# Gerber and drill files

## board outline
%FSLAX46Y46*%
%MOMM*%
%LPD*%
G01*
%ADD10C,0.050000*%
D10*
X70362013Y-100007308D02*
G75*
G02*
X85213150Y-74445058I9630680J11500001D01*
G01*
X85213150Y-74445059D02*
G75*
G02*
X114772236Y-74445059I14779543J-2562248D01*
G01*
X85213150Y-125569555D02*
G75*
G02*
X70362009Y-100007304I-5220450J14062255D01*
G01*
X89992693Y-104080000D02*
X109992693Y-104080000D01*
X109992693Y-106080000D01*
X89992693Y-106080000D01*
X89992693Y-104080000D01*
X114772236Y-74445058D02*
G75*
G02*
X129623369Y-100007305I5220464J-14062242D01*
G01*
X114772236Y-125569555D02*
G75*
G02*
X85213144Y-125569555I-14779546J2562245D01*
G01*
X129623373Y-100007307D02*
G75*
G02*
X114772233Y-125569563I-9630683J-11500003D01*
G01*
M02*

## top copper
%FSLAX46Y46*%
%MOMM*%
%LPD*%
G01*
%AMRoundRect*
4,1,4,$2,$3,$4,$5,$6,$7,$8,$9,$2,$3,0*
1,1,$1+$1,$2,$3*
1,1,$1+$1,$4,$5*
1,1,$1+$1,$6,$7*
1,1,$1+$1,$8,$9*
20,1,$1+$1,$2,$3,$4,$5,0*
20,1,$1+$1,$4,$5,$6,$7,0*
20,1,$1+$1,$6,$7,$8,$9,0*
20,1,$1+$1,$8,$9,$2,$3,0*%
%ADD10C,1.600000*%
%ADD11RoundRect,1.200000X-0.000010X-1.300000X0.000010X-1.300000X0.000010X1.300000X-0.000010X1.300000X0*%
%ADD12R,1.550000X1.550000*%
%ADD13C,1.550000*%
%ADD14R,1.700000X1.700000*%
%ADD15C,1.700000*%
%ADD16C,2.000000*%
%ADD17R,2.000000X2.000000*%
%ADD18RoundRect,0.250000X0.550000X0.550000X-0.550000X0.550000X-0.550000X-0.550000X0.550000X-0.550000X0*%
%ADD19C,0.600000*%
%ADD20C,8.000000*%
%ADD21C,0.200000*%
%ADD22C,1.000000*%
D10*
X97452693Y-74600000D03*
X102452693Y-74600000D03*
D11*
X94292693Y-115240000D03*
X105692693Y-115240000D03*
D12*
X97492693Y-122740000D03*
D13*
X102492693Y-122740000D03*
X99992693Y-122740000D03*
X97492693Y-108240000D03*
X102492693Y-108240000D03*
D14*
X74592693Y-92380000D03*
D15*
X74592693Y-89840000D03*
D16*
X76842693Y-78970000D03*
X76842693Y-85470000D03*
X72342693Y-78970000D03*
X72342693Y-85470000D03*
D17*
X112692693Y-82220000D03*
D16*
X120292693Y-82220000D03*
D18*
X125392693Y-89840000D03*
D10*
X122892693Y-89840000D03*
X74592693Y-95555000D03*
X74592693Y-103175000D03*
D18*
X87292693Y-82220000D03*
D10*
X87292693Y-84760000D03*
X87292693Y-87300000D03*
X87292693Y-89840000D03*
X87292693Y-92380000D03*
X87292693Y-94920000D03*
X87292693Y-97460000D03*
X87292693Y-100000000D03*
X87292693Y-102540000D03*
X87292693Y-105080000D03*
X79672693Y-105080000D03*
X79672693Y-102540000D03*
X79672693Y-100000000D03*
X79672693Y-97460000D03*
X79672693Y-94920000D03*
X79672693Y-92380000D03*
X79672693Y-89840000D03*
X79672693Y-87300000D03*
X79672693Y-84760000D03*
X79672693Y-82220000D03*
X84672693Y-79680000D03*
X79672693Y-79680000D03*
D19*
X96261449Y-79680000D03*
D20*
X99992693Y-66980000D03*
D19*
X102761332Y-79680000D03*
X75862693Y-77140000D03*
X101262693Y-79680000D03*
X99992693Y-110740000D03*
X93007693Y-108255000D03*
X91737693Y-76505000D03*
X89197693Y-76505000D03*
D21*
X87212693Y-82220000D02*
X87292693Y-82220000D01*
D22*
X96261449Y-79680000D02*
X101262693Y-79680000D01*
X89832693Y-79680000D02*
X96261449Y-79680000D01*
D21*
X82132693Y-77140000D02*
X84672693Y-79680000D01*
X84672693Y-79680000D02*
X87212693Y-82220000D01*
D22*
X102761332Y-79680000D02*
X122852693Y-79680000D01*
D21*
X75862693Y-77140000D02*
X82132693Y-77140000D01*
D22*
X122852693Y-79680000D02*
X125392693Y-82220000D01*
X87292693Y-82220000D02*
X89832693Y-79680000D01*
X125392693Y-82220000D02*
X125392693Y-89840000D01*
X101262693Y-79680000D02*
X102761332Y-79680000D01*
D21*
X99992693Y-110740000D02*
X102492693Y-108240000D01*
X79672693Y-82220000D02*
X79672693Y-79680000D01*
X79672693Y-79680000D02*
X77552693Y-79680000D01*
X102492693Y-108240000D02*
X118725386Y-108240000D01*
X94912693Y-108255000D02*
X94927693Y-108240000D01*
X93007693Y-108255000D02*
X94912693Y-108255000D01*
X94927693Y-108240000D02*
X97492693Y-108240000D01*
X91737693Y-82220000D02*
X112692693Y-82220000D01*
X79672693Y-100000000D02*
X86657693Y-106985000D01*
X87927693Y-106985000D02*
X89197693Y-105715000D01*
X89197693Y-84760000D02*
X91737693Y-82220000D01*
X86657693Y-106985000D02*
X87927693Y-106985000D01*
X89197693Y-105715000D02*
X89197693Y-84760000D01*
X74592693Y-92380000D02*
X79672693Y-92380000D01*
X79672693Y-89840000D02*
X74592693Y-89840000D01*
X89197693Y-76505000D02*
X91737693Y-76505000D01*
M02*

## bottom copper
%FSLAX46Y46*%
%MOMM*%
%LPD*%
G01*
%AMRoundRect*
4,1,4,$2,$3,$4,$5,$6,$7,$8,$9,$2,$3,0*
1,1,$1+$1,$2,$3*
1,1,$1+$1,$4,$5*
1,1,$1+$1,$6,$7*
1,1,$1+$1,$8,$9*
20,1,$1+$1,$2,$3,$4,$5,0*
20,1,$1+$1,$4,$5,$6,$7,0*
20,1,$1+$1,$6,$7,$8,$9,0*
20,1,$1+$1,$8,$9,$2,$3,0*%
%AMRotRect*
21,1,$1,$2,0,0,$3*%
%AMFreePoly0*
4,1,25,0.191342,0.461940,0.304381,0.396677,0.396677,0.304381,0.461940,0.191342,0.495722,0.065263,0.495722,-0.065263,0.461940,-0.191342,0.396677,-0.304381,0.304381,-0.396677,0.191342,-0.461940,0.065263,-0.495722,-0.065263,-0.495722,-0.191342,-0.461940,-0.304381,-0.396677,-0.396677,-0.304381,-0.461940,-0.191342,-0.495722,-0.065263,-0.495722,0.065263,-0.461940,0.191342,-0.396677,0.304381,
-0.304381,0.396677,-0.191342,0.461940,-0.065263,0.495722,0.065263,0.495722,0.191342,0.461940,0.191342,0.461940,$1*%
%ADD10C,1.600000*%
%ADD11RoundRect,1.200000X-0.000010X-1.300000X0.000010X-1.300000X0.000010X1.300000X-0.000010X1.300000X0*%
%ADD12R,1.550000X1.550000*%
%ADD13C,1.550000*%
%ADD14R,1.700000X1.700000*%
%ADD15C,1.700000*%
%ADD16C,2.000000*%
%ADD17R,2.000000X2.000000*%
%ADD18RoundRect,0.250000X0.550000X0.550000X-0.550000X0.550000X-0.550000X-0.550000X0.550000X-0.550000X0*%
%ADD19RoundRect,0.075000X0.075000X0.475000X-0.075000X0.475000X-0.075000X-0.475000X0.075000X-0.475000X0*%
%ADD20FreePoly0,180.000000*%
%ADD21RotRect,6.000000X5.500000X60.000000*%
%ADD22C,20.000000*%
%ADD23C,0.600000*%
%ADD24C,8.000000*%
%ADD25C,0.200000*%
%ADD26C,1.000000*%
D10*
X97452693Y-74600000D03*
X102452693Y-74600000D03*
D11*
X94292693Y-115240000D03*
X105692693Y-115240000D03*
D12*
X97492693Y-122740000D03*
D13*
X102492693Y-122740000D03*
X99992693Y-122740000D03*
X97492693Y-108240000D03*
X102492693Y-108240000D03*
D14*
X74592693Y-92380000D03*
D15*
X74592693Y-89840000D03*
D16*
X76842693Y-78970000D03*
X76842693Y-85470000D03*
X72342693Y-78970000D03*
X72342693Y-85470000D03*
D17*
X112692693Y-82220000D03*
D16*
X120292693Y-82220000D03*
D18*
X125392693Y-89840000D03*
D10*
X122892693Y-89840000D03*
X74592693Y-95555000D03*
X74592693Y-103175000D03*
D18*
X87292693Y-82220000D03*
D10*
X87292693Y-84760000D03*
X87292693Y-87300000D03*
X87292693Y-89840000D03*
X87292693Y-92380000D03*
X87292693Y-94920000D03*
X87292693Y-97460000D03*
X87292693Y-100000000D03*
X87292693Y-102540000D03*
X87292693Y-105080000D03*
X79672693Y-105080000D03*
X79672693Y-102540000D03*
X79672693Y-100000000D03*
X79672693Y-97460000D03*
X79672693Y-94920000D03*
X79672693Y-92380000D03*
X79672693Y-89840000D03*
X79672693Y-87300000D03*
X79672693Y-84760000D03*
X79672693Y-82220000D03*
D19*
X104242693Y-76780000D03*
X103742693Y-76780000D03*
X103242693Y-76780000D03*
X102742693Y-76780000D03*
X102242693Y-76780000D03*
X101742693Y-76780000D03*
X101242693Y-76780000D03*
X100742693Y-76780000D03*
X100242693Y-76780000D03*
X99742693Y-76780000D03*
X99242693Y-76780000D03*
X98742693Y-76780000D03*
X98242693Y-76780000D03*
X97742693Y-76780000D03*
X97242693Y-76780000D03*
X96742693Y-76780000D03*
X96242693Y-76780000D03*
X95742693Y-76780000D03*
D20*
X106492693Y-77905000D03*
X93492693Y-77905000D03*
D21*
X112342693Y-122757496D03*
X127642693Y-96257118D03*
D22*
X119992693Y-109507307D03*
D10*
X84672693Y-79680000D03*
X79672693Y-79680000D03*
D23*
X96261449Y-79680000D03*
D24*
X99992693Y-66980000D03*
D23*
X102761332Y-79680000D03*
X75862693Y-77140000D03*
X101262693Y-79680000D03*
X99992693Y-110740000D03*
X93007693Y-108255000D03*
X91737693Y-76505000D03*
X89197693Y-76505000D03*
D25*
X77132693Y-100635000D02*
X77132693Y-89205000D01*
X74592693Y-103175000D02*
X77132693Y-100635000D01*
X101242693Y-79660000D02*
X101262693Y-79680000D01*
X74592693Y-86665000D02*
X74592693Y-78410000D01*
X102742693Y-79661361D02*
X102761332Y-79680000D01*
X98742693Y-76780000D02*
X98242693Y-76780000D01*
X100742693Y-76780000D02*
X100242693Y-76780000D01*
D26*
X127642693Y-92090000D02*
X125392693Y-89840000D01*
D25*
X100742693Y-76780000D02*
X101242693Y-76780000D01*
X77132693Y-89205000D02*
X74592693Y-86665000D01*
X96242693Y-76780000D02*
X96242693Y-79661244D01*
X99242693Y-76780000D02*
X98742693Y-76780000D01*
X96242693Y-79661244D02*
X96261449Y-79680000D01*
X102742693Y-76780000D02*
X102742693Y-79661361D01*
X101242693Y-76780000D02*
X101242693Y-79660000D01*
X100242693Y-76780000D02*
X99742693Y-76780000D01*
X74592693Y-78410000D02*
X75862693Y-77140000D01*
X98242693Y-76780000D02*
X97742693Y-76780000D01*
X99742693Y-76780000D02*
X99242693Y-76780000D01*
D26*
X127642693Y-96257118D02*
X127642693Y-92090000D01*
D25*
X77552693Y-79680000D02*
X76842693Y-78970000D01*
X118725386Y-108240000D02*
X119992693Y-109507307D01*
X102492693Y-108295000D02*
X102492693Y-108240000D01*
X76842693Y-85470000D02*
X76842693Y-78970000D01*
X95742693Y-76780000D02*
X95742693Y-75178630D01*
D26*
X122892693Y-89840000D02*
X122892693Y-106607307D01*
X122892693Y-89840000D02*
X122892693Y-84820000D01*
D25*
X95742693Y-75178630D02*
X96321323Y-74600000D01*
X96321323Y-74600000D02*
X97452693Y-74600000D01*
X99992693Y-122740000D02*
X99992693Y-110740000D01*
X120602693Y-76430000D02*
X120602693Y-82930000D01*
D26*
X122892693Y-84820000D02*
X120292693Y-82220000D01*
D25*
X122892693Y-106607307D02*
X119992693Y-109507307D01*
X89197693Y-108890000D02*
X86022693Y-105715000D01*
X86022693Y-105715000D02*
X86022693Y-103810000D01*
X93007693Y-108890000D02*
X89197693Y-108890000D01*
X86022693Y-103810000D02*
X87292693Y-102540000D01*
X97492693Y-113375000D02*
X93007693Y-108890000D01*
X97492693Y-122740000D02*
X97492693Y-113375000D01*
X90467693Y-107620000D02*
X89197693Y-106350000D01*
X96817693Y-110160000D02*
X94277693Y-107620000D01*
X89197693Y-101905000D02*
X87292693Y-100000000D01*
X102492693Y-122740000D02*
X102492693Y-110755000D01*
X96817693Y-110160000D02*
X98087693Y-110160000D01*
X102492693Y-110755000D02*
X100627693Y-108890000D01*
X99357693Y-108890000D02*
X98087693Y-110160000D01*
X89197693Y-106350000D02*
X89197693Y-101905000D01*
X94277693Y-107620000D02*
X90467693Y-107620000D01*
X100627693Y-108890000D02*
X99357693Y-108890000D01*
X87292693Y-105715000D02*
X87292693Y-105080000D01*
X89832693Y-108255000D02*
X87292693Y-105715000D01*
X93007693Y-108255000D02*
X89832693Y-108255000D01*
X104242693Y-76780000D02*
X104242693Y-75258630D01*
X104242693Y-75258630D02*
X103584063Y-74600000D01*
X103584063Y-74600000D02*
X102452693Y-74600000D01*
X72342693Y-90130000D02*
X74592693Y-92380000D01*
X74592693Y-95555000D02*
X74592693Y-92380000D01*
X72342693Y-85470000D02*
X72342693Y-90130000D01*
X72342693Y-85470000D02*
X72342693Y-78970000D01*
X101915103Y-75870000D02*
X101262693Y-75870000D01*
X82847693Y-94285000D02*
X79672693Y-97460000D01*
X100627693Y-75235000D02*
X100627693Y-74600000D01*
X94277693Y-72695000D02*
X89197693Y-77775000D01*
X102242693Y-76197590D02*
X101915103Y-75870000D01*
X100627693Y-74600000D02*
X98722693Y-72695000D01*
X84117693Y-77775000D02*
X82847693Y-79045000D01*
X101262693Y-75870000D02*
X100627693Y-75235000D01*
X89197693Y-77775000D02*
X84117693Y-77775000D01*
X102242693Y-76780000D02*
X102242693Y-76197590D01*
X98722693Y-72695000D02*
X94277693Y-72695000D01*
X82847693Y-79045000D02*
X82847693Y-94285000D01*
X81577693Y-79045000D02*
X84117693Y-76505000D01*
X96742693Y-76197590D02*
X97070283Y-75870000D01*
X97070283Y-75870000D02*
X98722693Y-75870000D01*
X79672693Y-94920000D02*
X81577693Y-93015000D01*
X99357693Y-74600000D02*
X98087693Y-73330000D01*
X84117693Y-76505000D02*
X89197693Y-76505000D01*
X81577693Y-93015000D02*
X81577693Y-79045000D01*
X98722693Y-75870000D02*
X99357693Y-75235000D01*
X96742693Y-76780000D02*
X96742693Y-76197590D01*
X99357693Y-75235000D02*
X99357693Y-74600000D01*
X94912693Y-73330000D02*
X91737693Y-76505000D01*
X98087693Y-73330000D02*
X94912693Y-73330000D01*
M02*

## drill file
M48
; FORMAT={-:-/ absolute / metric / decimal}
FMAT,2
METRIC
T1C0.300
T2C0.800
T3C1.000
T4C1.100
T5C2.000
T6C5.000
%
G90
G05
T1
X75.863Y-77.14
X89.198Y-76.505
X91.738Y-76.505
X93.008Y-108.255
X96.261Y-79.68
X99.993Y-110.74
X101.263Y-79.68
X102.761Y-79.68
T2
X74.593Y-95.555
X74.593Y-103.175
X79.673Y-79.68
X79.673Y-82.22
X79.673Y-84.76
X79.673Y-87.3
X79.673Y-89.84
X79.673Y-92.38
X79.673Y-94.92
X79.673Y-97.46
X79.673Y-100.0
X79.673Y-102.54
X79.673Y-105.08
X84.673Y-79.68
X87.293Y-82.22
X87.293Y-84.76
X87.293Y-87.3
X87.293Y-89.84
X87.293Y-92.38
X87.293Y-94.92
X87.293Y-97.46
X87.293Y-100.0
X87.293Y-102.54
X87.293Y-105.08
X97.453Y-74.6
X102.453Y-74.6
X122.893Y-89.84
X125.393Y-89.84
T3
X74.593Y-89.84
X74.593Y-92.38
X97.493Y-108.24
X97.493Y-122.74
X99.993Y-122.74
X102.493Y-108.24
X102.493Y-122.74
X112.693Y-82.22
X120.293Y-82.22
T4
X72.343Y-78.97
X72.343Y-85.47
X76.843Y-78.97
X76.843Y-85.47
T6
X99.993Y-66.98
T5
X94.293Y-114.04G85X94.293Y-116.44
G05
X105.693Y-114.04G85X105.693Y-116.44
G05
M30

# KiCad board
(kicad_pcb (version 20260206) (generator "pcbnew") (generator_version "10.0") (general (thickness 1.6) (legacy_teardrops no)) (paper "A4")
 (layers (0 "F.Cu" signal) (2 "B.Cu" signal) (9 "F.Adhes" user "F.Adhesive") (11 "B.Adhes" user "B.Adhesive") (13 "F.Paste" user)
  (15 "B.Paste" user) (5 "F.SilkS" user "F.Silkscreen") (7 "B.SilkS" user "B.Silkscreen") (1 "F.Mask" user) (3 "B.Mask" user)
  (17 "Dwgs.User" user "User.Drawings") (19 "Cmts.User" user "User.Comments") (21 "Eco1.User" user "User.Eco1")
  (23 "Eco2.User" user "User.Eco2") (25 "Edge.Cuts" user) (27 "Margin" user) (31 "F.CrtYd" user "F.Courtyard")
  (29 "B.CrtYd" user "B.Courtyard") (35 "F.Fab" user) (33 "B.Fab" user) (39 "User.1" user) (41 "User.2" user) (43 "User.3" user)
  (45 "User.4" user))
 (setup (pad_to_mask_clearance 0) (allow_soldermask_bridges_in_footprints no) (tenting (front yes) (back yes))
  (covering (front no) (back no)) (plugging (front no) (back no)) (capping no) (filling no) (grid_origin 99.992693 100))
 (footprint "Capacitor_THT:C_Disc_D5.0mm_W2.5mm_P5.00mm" (layer "F.Cu") (at 97.452693 74.6)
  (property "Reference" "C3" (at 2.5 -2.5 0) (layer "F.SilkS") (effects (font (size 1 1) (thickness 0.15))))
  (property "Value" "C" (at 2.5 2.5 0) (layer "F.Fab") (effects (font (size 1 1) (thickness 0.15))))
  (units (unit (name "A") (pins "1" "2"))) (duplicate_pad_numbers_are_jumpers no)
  (pad "1" thru_hole circle (at 0 0) (size 1.6 1.6) (drill 0.8) (layers "*.Cu" "*.Mask") (remove_unused_layers no) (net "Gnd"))
  (pad "2" thru_hole circle (at 5 0) (size 1.6 1.6) (drill 0.8) (layers "*.Cu" "*.Mask") (remove_unused_layers no) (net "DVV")))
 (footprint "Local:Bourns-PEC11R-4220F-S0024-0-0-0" (layer "F.Cu") (at 99.992693 115.24)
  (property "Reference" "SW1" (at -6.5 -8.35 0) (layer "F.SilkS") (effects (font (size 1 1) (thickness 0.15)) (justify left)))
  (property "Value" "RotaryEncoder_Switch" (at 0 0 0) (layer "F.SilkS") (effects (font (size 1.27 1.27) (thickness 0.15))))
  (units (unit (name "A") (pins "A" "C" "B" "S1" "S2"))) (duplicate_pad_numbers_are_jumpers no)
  (pad "3" thru_hole roundrect (at -5.7 0) (size 2.4 5) (drill oval 2 4.4) (layers "*.Cu" "*.Mask") (remove_unused_layers no)
   (roundrect_rratio 0.5))
  (pad "4" thru_hole roundrect (at 5.7 0) (size 2.4 5) (drill oval 2 4.4) (layers "*.Cu" "*.Mask") (remove_unused_layers no)
   (roundrect_rratio 0.5))
  (pad "A" thru_hole rect (at -2.5 7.5) (size 1.55 1.55) (drill 1) (layers "*.Cu" "*.Mask") (remove_unused_layers no) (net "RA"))
  (pad "B" thru_hole circle (at 2.5 7.5) (size 1.55 1.55) (drill 1) (layers "*.Cu" "*.Mask") (remove_unused_layers no) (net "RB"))
  (pad "C" thru_hole circle (at 0 7.5) (size 1.55 1.55) (drill 1) (layers "*.Cu" "*.Mask") (remove_unused_layers no) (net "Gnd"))
  (pad "S1" thru_hole circle (at -2.5 -7) (size 1.55 1.55) (drill 1) (layers "*.Cu" "*.Mask") (remove_unused_layers no) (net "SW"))
  (pad "S2" thru_hole circle (at 2.5 -7) (size 1.55 1.55) (drill 1) (layers "*.Cu" "*.Mask") (remove_unused_layers no) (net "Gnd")))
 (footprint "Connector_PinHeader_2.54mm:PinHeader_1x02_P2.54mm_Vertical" (layer "F.Cu") (at 74.592693 92.38 180)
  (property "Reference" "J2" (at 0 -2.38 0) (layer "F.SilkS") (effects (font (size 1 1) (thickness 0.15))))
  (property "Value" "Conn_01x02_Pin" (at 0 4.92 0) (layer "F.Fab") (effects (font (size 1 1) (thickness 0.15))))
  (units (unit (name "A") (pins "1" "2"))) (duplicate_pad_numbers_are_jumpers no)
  (pad "1" thru_hole rect (at 0 0 180) (size 1.7 1.7) (drill 1) (layers "*.Cu" "*.Mask") (remove_unused_layers no) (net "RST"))
  (pad "2" thru_hole circle (at 0 2.54 180) (size 1.7 1.7) (drill 1) (layers "*.Cu" "*.Mask") (remove_unused_layers no) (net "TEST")))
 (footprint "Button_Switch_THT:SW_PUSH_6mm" (layer "F.Cu") (at 76.842693 78.97 -90)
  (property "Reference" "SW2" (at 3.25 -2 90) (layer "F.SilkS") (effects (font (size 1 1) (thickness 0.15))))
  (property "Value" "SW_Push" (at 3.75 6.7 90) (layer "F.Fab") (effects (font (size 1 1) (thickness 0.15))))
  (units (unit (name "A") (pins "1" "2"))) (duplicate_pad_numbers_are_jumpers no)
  (pad "1" thru_hole circle (at 0 0) (size 2 2) (drill 1.1) (layers "*.Cu" "*.Mask") (remove_unused_layers no) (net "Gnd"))
  (pad "1" thru_hole circle (at 6.5 0) (size 2 2) (drill 1.1) (layers "*.Cu" "*.Mask") (remove_unused_layers no) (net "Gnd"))
  (pad "2" thru_hole circle (at 0 4.5) (size 2 2) (drill 1.1) (layers "*.Cu" "*.Mask") (remove_unused_layers no) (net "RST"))
  (pad "2" thru_hole circle (at 6.5 4.5) (size 2 2) (drill 1.1) (layers "*.Cu" "*.Mask") (remove_unused_layers no) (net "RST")))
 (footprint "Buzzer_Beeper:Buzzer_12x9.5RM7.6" (layer "F.Cu") (at 112.692693 82.22)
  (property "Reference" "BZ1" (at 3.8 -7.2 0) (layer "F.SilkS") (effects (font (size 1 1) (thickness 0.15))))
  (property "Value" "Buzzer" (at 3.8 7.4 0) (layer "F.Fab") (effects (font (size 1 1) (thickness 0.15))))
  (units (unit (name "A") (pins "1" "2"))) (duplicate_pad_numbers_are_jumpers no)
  (pad "1" thru_hole rect (at 0 0) (size 2 2) (drill 1) (layers "*.Cu" "*.Mask") (remove_unused_layers no) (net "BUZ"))
  (pad "2" thru_hole circle (at 7.6 0) (size 2 2) (drill 1) (layers "*.Cu" "*.Mask") (remove_unused_layers no) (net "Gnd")))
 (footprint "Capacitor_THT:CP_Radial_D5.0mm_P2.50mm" (layer "F.Cu") (at 125.392693 89.84 180)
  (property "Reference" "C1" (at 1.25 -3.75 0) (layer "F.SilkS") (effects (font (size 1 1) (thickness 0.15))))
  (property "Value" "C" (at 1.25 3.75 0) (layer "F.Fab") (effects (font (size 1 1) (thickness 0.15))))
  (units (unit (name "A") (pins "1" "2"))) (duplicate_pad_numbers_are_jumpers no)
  (pad "1" thru_hole roundrect (at 0 0 180) (size 1.6 1.6) (drill 0.8) (layers "*.Cu" "*.Mask") (remove_unused_layers no)
   (roundrect_rratio 0.15625) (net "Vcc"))
  (pad "2" thru_hole circle (at 2.5 0 180) (size 1.6 1.6) (drill 0.8) (layers "*.Cu" "*.Mask") (remove_unused_layers no) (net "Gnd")))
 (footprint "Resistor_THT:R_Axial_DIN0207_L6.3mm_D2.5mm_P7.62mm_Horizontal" (layer "F.Cu") (at 74.592693 95.555 -90)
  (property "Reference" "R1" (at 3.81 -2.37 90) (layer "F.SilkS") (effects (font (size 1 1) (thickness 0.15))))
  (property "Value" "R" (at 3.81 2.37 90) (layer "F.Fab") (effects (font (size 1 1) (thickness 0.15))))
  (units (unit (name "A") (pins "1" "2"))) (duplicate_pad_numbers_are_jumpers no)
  (pad "1" thru_hole circle (at 0 0 270) (size 1.6 1.6) (drill 0.8) (layers "*.Cu" "*.Mask") (remove_unused_layers no) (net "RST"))
  (pad "2" thru_hole circle (at 7.62 0 270) (size 1.6 1.6) (drill 0.8) (layers "*.Cu" "*.Mask") (remove_unused_layers no) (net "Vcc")))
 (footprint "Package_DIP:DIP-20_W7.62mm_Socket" (layer "B.Cu") (at 87.292693 82.22 180)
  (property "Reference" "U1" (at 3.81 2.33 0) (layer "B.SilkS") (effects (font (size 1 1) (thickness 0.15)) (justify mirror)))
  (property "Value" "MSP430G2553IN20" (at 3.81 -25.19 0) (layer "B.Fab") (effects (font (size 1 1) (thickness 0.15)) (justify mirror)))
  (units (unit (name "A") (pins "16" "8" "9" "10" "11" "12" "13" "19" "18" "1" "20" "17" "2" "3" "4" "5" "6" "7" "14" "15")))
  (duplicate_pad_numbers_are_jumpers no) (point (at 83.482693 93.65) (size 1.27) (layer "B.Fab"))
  (pad "1" thru_hole roundrect (at 0 0 180) (size 1.6 1.6) (drill 0.8) (layers "*.Cu" "*.Mask") (remove_unused_layers no)
   (roundrect_rratio 0.15625) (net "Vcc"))
  (pad "2" thru_hole circle (at 0 -2.54 180) (size 1.6 1.6) (drill 0.8) (layers "*.Cu" "*.Mask") (remove_unused_layers no)
   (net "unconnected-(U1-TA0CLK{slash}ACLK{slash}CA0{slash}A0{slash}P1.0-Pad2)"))
  (pad "3" thru_hole circle (at 0 -5.08 180) (size 1.6 1.6) (drill 0.8) (layers "*.Cu" "*.Mask") (remove_unused_layers no)
   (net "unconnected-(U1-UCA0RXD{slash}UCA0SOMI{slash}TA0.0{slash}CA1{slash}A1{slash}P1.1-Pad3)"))
  (pad "4" thru_hole circle (at 0 -7.62 180) (size 1.6 1.6) (drill 0.8) (layers "*.Cu" "*.Mask") (remove_unused_layers no) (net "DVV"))
  (pad "5" thru_hole circle (at 0 -10.16 180) (size 1.6 1.6) (drill 0.8) (layers "*.Cu" "*.Mask") (remove_unused_layers no) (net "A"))
  (pad "6" thru_hole circle (at 0 -12.7 180) (size 1.6 1.6) (drill 0.8) (layers "*.Cu" "*.Mask") (remove_unused_layers no) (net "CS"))
  (pad "7" thru_hole circle (at 0 -15.24 180) (size 1.6 1.6) (drill 0.8) (layers "*.Cu" "*.Mask") (remove_unused_layers no) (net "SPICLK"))
  (pad "8" thru_hole circle (at 0 -17.78 180) (size 1.6 1.6) (drill 0.8) (layers "*.Cu" "*.Mask") (remove_unused_layers no) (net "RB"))
  (pad "9" thru_hole circle (at 0 -20.32 180) (size 1.6 1.6) (drill 0.8) (layers "*.Cu" "*.Mask") (remove_unused_layers no) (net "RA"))
  (pad "10" thru_hole circle (at 0 -22.86 180) (size 1.6 1.6) (drill 0.8) (layers "*.Cu" "*.Mask") (remove_unused_layers no) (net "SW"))
  (pad "11" thru_hole circle (at 7.62 -22.86 180) (size 1.6 1.6) (drill 0.8) (layers "*.Cu" "*.Mask") (remove_unused_layers no)
   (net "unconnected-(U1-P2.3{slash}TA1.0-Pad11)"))
  (pad "12" thru_hole circle (at 7.62 -20.32 180) (size 1.6 1.6) (drill 0.8) (layers "*.Cu" "*.Mask") (remove_unused_layers no)
   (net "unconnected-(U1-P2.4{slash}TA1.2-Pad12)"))
  (pad "13" thru_hole circle (at 7.62 -17.78 180) (size 1.6 1.6) (drill 0.8) (layers "*.Cu" "*.Mask") (remove_unused_layers no) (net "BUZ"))
  (pad "14" thru_hole circle (at 7.62 -15.24 180) (size 1.6 1.6) (drill 0.8) (layers "*.Cu" "*.Mask") (remove_unused_layers no) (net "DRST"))
  (pad "15" thru_hole circle (at 7.62 -12.7 180) (size 1.6 1.6) (drill 0.8) (layers "*.Cu" "*.Mask") (remove_unused_layers no) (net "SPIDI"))
  (pad "16" thru_hole circle (at 7.62 -10.16 180) (size 1.6 1.6) (drill 0.8) (layers "*.Cu" "*.Mask") (remove_unused_layers no) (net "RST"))
  (pad "17" thru_hole circle (at 7.62 -7.62 180) (size 1.6 1.6) (drill 0.8) (layers "*.Cu" "*.Mask") (remove_unused_layers no) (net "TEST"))
  (pad "18" thru_hole circle (at 7.62 -5.08 180) (size 1.6 1.6) (drill 0.8) (layers "*.Cu" "*.Mask") (remove_unused_layers no)
   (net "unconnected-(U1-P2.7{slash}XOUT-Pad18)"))
  (pad "19" thru_hole circle (at 7.62 -2.54 180) (size 1.6 1.6) (drill 0.8) (layers "*.Cu" "*.Mask") (remove_unused_layers no)
   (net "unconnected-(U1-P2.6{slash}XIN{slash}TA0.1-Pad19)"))
  (pad "20" thru_hole circle (at 7.62 0 180) (size 1.6 1.6) (drill 0.8) (layers "*.Cu" "*.Mask") (remove_unused_layers no) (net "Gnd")))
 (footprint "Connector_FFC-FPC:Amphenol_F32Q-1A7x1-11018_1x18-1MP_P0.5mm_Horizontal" (layer "B.Cu") (at 99.992693 79.68 180)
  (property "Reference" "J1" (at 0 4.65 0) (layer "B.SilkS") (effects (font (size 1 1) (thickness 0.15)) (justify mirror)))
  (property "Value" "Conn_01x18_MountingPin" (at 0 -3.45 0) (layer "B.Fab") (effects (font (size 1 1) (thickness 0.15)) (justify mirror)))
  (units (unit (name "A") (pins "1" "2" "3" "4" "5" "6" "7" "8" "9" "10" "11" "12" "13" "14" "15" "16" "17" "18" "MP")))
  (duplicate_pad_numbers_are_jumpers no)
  (pad "1" smd roundrect (at -4.25 2.9 180) (size 0.3 1.1) (layers "B.Cu" "B.Mask" "B.Paste") (roundrect_rratio 0.25) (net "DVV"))
  (pad "2" smd roundrect (at -3.75 2.9 180) (size 0.3 1.1) (layers "B.Cu" "B.Mask" "B.Paste") (roundrect_rratio 0.25) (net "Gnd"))
  (pad "3" smd roundrect (at -3.25 2.9 180) (size 0.3 1.1) (layers "B.Cu" "B.Mask" "B.Paste") (roundrect_rratio 0.25) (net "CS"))
  (pad "4" smd roundrect (at -2.75 2.9 180) (size 0.3 1.1) (layers "B.Cu" "B.Mask" "B.Paste") (roundrect_rratio 0.25) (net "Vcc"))
  (pad "5" smd roundrect (at -2.25 2.9 180) (size 0.3 1.1) (layers "B.Cu" "B.Mask" "B.Paste") (roundrect_rratio 0.25) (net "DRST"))
  (pad "6" smd roundrect (at -1.75 2.9 180) (size 0.3 1.1) (layers "B.Cu" "B.Mask" "B.Paste") (roundrect_rratio 0.25) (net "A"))
  (pad "7" smd roundrect (at -1.25 2.9 180) (size 0.3 1.1) (layers "B.Cu" "B.Mask" "B.Paste") (roundrect_rratio 0.25) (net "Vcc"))
  (pad "8" smd roundrect (at -0.75 2.9 180) (size 0.3 1.1) (layers "B.Cu" "B.Mask" "B.Paste") (roundrect_rratio 0.25) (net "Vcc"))
  (pad "9" smd roundrect (at -0.25 2.9 180) (size 0.3 1.1) (layers "B.Cu" "B.Mask" "B.Paste") (roundrect_rratio 0.25) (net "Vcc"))
  (pad "10" smd roundrect (at 0.25 2.9 180) (size 0.3 1.1) (layers "B.Cu" "B.Mask" "B.Paste") (roundrect_rratio 0.25) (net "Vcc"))
  (pad "11" smd roundrect (at 0.75 2.9 180) (size 0.3 1.1) (layers "B.Cu" "B.Mask" "B.Paste") (roundrect_rratio 0.25) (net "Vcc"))
  (pad "12" smd roundrect (at 1.25 2.9 180) (size 0.3 1.1) (layers "B.Cu" "B.Mask" "B.Paste") (roundrect_rratio 0.25) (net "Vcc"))
  (pad "13" smd roundrect (at 1.75 2.9 180) (size 0.3 1.1) (layers "B.Cu" "B.Mask" "B.Paste") (roundrect_rratio 0.25) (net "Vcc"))
  (pad "14" smd roundrect (at 2.25 2.9 180) (size 0.3 1.1) (layers "B.Cu" "B.Mask" "B.Paste") (roundrect_rratio 0.25) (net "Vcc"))
  (pad "15" smd roundrect (at 2.75 2.9 180) (size 0.3 1.1) (layers "B.Cu" "B.Mask" "B.Paste") (roundrect_rratio 0.25) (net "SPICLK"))
  (pad "16" smd roundrect (at 3.25 2.9 180) (size 0.3 1.1) (layers "B.Cu" "B.Mask" "B.Paste") (roundrect_rratio 0.25) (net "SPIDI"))
  (pad "17" smd roundrect (at 3.75 2.9 180) (size 0.3 1.1) (layers "B.Cu" "B.Mask" "B.Paste") (roundrect_rratio 0.25) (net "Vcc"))
  (pad "18" smd roundrect (at 4.25 2.9 180) (size 0.3 1.1) (layers "B.Cu" "B.Mask" "B.Paste") (roundrect_rratio 0.25) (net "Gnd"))
  (pad "MP" smd custom (at -6.5 1.775 180) (size 1 1) (layers "B.Cu" "B.Mask" "B.Paste") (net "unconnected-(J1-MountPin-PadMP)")
   (options (clearance outline) (anchor circle)) (primitives))
  (pad "MP" smd custom (at 6.5 1.775 180) (size 1 1) (layers "B.Cu" "B.Mask" "B.Paste") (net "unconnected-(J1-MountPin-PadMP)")
   (options (clearance outline) (anchor circle)) (primitives)))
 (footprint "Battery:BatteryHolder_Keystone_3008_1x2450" (layer "B.Cu") (at 119.992693 109.507307 60)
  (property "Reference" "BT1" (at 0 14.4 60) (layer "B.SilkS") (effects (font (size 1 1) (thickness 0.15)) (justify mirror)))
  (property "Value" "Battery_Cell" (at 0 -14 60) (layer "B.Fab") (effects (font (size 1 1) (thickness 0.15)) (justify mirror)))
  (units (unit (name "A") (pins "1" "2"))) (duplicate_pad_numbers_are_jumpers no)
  (pad "1" smd rect (at -15.3 0 60) (size 6 5.5) (layers "B.Cu" "B.Mask" "B.Paste") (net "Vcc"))
  (pad "1" smd rect (at 15.3 0 60) (size 6 5.5) (layers "B.Cu" "B.Mask" "B.Paste") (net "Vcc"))
  (pad "2" smd circle (at 0 0 60) (size 20 20) (layers "B.Cu" "B.Mask") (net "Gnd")))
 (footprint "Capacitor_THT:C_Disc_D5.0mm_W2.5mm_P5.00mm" (layer "B.Cu") (at 84.672693 79.68 180)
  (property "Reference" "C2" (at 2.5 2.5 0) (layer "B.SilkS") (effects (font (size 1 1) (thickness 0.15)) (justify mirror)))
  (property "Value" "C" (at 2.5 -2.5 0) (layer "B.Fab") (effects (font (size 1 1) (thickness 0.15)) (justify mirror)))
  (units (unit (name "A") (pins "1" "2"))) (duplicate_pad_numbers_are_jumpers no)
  (pad "1" thru_hole circle (at 0 0 180) (size 1.6 1.6) (drill 0.8) (layers "*.Cu" "*.Mask") (remove_unused_layers no) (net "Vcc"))
  (pad "2" thru_hole circle (at 5 0 180) (size 1.6 1.6) (drill 0.8) (layers "*.Cu" "*.Mask") (remove_unused_layers no) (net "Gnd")))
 (gr_arc (start 70.362013 100.007308) (mid 67.02274 80.972034) (end 85.21315 74.445058) (stroke (width 0.05) (type solid))
  (layer "Edge.Cuts"))
 (gr_arc (start 85.21315 74.445059) (mid 99.992693 62.007307) (end 114.772236 74.445059) (stroke (width 0.05) (type solid))
  (layer "Edge.Cuts"))
 (gr_arc (start 85.21315 125.569555) (mid 67.022742 119.042581) (end 70.362012 100.007307) (stroke (width 0.05) (type solid))
  (layer "Edge.Cuts"))
 (gr_rect (start 89.992693 104.08) (end 109.992693 106.08) (stroke (width 0.05) (type solid)) (fill no) (layer "Edge.Cuts"))
 (gr_arc (start 114.772236 74.445058) (mid 132.962646 80.972034) (end 129.623373 100.007309) (stroke (width 0.05) (type solid))
  (layer "Edge.Cuts"))
 (gr_arc (start 114.772236 125.569555) (mid 99.992693 138.007307) (end 85.21315 125.569554) (stroke (width 0.05) (type solid))
  (layer "Edge.Cuts"))
 (gr_arc (start 129.623373 100.007307) (mid 132.962645 119.042581) (end 114.772236 125.569555) (stroke (width 0.05) (type solid))
  (layer "Edge.Cuts"))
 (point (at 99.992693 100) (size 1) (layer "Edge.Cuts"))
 (segment (start 87.212693 82.22) (end 87.292693 82.22) (width 0.2) (layer "F.Cu") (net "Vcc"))
 (segment (start 96.261449 79.68) (end 101.262693 79.68) (width 1) (layer "F.Cu") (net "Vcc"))
 (segment (start 89.832693 79.68) (end 96.261449 79.68) (width 1) (layer "F.Cu") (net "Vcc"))
 (segment (start 82.132693 77.14) (end 84.672693 79.68) (width 0.2) (layer "F.Cu") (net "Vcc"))
 (segment (start 84.672693 79.68) (end 87.212693 82.22) (width 0.2) (layer "F.Cu") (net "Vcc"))
 (segment (start 102.761332 79.68) (end 122.852693 79.68) (width 1) (layer "F.Cu") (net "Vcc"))
 (segment (start 75.862693 77.14) (end 82.132693 77.14) (width 0.2) (layer "F.Cu") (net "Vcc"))
 (segment (start 122.852693 79.68) (end 125.392693 82.22) (width 1) (layer "F.Cu") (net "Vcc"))
 (segment (start 87.292693 82.22) (end 89.832693 79.68) (width 1) (layer "F.Cu") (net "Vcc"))
 (segment (start 125.392693 82.22) (end 125.392693 89.84) (width 1) (layer "F.Cu") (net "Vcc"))
 (segment (start 101.262693 79.68) (end 102.761332 79.68) (width 1) (layer "F.Cu") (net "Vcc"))
 (via (at 96.261449 79.68) (size 0.6) (drill 0.3) (layers "F.Cu" "B.Cu") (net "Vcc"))
 (via (at 99.992693 66.98) (size 8) (drill 5) (layers "F.Cu" "B.Cu") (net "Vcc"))
 (via (at 102.761332 79.68) (size 0.6) (drill 0.3) (layers "F.Cu" "B.Cu") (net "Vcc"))
 (via (at 75.862693 77.14) (size 0.6) (drill 0.3) (layers "F.Cu" "B.Cu") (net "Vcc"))
 (via (at 101.262693 79.68) (size 0.6) (drill 0.3) (layers "F.Cu" "B.Cu") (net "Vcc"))
 (segment (start 77.132693 100.635) (end 77.132693 89.205) (width 0.2) (layer "B.Cu") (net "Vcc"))
 (segment (start 74.592693 103.175) (end 77.132693 100.635) (width 0.2) (layer "B.Cu") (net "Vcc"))
 (segment (start 101.242693 79.66) (end 101.262693 79.68) (width 0.2) (layer "B.Cu") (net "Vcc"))
 (segment (start 74.592693 86.665) (end 74.592693 78.41) (width 0.2) (layer "B.Cu") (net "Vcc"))
 (segment (start 102.742693 79.661361) (end 102.761332 79.68) (width 0.2) (layer "B.Cu") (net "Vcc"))
 (segment (start 98.742693 76.78) (end 98.242693 76.78) (width 0.2) (layer "B.Cu") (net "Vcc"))
 (segment (start 100.742693 76.78) (end 100.242693 76.78) (width 0.2) (layer "B.Cu") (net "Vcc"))
 (segment (start 127.642693 92.09) (end 125.392693 89.84) (width 1) (layer "B.Cu") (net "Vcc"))
 (segment (start 100.742693 76.78) (end 101.242693 76.78) (width 0.2) (layer "B.Cu") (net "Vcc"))
 (segment (start 77.132693 89.205) (end 74.592693 86.665) (width 0.2) (layer "B.Cu") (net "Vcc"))
 (segment (start 96.242693 76.78) (end 96.242693 79.661244) (width 0.2) (layer "B.Cu") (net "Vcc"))
 (segment (start 99.242693 76.78) (end 98.742693 76.78) (width 0.2) (layer "B.Cu") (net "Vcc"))
 (segment (start 96.242693 79.661244) (end 96.261449 79.68) (width 0.2) (layer "B.Cu") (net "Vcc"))
 (segment (start 102.742693 76.78) (end 102.742693 79.661361) (width 0.2) (layer "B.Cu") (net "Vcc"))
 (segment (start 101.242693 76.78) (end 101.242693 79.66) (width 0.2) (layer "B.Cu") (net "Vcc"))
 (segment (start 100.242693 76.78) (end 99.742693 76.78) (width 0.2) (layer "B.Cu") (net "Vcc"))
 (segment (start 74.592693 78.41) (end 75.862693 77.14) (width 0.2) (layer "B.Cu") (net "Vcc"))
 (segment (start 98.242693 76.78) (end 97.742693 76.78) (width 0.2) (layer "B.Cu") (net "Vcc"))
 (segment (start 99.742693 76.78) (end 99.242693 76.78) (width 0.2) (layer "B.Cu") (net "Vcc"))
 (segment (start 127.642693 96.257118) (end 127.642693 92.09) (width 1) (layer "B.Cu") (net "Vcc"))
 (segment (start 99.992693 110.74) (end 102.492693 108.24) (width 0.2) (layer "F.Cu") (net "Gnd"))
 (segment (start 79.672693 82.22) (end 79.672693 79.68) (width 0.2) (layer "F.Cu") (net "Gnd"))
 (segment (start 79.672693 79.68) (end 77.552693 79.68) (width 0.2) (layer "F.Cu") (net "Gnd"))
 (segment (start 102.492693 108.24) (end 118.725386 108.24) (width 0.2) (layer "F.Cu") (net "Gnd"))
 (via (at 99.992693 110.74) (size 0.6) (drill 0.3) (layers "F.Cu" "B.Cu") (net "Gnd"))
 (segment (start 77.552693 79.68) (end 76.842693 78.97) (width 0.2) (layer "B.Cu") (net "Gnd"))
 (segment (start 118.725386 108.24) (end 119.992693 109.507307) (width 0.2) (layer "B.Cu") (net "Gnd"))
 (segment (start 102.492693 108.295) (end 102.492693 108.24) (width 0.2) (layer "B.Cu") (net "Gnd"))
 (segment (start 76.842693 85.47) (end 76.842693 78.97) (width 0.2) (layer "B.Cu") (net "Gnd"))
 (segment (start 95.742693 76.78) (end 95.742693 75.17863) (width 0.2) (layer "B.Cu") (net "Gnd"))
 (segment (start 122.892693 89.84) (end 122.892693 106.607307) (width 1) (layer "B.Cu") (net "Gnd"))
 (segment (start 122.892693 89.84) (end 122.892693 84.82) (width 1) (layer "B.Cu") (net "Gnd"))
 (segment (start 95.742693 75.17863) (end 96.321323 74.6) (width 0.2) (layer "B.Cu") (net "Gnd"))
 (segment (start 96.321323 74.6) (end 97.452693 74.6) (width 0.2) (layer "B.Cu") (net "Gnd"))
 (segment (start 99.992693 122.74) (end 99.992693 110.74) (width 0.2) (layer "B.Cu") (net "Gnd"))
 (segment (start 120.602693 76.43) (end 120.602693 82.93) (width 0.2) (layer "B.Cu") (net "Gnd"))
 (segment (start 122.892693 84.82) (end 120.292693 82.22) (width 1) (layer "B.Cu") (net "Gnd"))
 (segment (start 122.892693 106.607307) (end 119.992693 109.507307) (width 0.2) (layer "B.Cu") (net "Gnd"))
 (segment (start 89.197693 108.89) (end 86.022693 105.715) (width 0.2) (layer "B.Cu") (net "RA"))
 (segment (start 86.022693 105.715) (end 86.022693 103.81) (width 0.2) (layer "B.Cu") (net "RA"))
 (segment (start 93.007693 108.89) (end 89.197693 108.89) (width 0.2) (layer "B.Cu") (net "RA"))
 (segment (start 86.022693 103.81) (end 87.292693 102.54) (width 0.2) (layer "B.Cu") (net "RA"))
 (segment (start 97.492693 113.375) (end 93.007693 108.89) (width 0.2) (layer "B.Cu") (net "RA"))
 (segment (start 97.492693 122.74) (end 97.492693 113.375) (width 0.2) (layer "B.Cu") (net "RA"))
 (segment (start 90.467693 107.62) (end 89.197693 106.35) (width 0.2) (layer "B.Cu") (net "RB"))
 (segment (start 96.817693 110.16) (end 94.277693 107.62) (width 0.2) (layer "B.Cu") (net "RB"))
 (segment (start 89.197693 101.905) (end 87.292693 100) (width 0.2) (layer "B.Cu") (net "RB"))
 (segment (start 102.492693 122.74) (end 102.492693 110.755) (width 0.2) (layer "B.Cu") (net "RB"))
 (segment (start 96.817693 110.16) (end 98.087693 110.16) (width 0.2) (layer "B.Cu") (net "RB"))
 (segment (start 102.492693 110.755) (end 100.627693 108.89) (width 0.2) (layer "B.Cu") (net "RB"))
 (segment (start 99.357693 108.89) (end 98.087693 110.16) (width 0.2) (layer "B.Cu") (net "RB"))
 (segment (start 89.197693 106.35) (end 89.197693 101.905) (width 0.2) (layer "B.Cu") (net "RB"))
 (segment (start 94.277693 107.62) (end 90.467693 107.62) (width 0.2) (layer "B.Cu") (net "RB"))
 (segment (start 100.627693 108.89) (end 99.357693 108.89) (width 0.2) (layer "B.Cu") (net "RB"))
 (segment (start 94.912693 108.255) (end 94.927693 108.24) (width 0.2) (layer "F.Cu") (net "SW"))
 (segment (start 93.007693 108.255) (end 94.912693 108.255) (width 0.2) (layer "F.Cu") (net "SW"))
 (segment (start 94.927693 108.24) (end 97.492693 108.24) (width 0.2) (layer "F.Cu") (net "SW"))
 (via (at 93.007693 108.255) (size 0.6) (drill 0.3) (layers "F.Cu" "B.Cu") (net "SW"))
 (segment (start 87.292693 105.715) (end 87.292693 105.08) (width 0.2) (layer "B.Cu") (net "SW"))
 (segment (start 89.832693 108.255) (end 87.292693 105.715) (width 0.2) (layer "B.Cu") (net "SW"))
 (segment (start 93.007693 108.255) (end 89.832693 108.255) (width 0.2) (layer "B.Cu") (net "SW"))
 (segment (start 104.242693 76.78) (end 104.242693 75.25863) (width 0.2) (layer "B.Cu") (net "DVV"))
 (segment (start 104.242693 75.25863) (end 103.584063 74.6) (width 0.2) (layer "B.Cu") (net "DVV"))
 (segment (start 103.584063 74.6) (end 102.452693 74.6) (width 0.2) (layer "B.Cu") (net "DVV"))
 (segment (start 91.737693 82.22) (end 112.692693 82.22) (width 0.2) (layer "F.Cu") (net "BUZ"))
 (segment (start 79.672693 100) (end 86.657693 106.985) (width 0.2) (layer "F.Cu") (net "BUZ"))
 (segment (start 87.927693 106.985) (end 89.197693 105.715) (width 0.2) (layer "F.Cu") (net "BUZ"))
 (segment (start 89.197693 84.76) (end 91.737693 82.22) (width 0.2) (layer "F.Cu") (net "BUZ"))
 (segment (start 86.657693 106.985) (end 87.927693 106.985) (width 0.2) (layer "F.Cu") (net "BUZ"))
 (segment (start 89.197693 105.715) (end 89.197693 84.76) (width 0.2) (layer "F.Cu") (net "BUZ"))
 (segment (start 74.592693 92.38) (end 79.672693 92.38) (width 0.2) (layer "F.Cu") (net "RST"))
 (segment (start 72.342693 90.13) (end 74.592693 92.38) (width 0.2) (layer "B.Cu") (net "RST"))
 (segment (start 74.592693 95.555) (end 74.592693 92.38) (width 0.2) (layer "B.Cu") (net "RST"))
 (segment (start 72.342693 85.47) (end 72.342693 90.13) (width 0.2) (layer "B.Cu") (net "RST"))
 (segment (start 72.342693 85.47) (end 72.342693 78.97) (width 0.2) (layer "B.Cu") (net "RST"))
 (segment (start 79.672693 89.84) (end 74.592693 89.84) (width 0.2) (layer "F.Cu") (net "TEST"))
 (segment (start 101.915103 75.87) (end 101.262693 75.87) (width 0.2) (layer "B.Cu") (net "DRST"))
 (segment (start 82.847693 94.285) (end 79.672693 97.46) (width 0.2) (layer "B.Cu") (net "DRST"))
 (segment (start 100.627693 75.235) (end 100.627693 74.6) (width 0.2) (layer "B.Cu") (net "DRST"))
 (segment (start 94.277693 72.695) (end 89.197693 77.775) (width 0.2) (layer "B.Cu") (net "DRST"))
 (segment (start 102.242693 76.19759) (end 101.915103 75.87) (width 0.2) (layer "B.Cu") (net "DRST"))
 (segment (start 100.627693 74.6) (end 98.722693 72.695) (width 0.2) (layer "B.Cu") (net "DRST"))
 (segment (start 84.117693 77.775) (end 82.847693 79.045) (width 0.2) (layer "B.Cu") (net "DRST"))
 (segment (start 101.262693 75.87) (end 100.627693 75.235) (width 0.2) (layer "B.Cu") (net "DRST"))
 (segment (start 89.197693 77.775) (end 84.117693 77.775) (width 0.2) (layer "B.Cu") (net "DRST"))
 (segment (start 102.242693 76.78) (end 102.242693 76.19759) (width 0.2) (layer "B.Cu") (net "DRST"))
 (segment (start 98.722693 72.695) (end 94.277693 72.695) (width 0.2) (layer "B.Cu") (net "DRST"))
 (segment (start 82.847693 79.045) (end 82.847693 94.285) (width 0.2) (layer "B.Cu") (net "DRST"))
 (segment (start 89.197693 76.505) (end 91.737693 76.505) (width 0.2) (layer "F.Cu") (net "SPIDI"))
 (via (at 91.737693 76.505) (size 0.6) (drill 0.3) (layers "F.Cu" "B.Cu") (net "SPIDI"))
 (via (at 89.197693 76.505) (size 0.6) (drill 0.3) (layers "F.Cu" "B.Cu") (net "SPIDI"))
 (segment (start 81.577693 79.045) (end 84.117693 76.505) (width 0.2) (layer "B.Cu") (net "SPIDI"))
 (segment (start 96.742693 76.19759) (end 97.070283 75.87) (width 0.2) (layer "B.Cu") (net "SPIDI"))
 (segment (start 97.070283 75.87) (end 98.722693 75.87) (width 0.2) (layer "B.Cu") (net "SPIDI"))
 (segment (start 79.672693 94.92) (end 81.577693 93.015) (width 0.2) (layer "B.Cu") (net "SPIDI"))
 (segment (start 99.357693 74.6) (end 98.087693 73.33) (width 0.2) (layer "B.Cu") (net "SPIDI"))
 (segment (start 84.117693 76.505) (end 89.197693 76.505) (width 0.2) (layer "B.Cu") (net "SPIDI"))
 (segment (start 81.577693 93.015) (end 81.577693 79.045) (width 0.2) (layer "B.Cu") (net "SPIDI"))
 (segment (start 98.722693 75.87) (end 99.357693 75.235) (width 0.2) (layer "B.Cu") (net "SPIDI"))
 (segment (start 96.742693 76.78) (end 96.742693 76.19759) (width 0.2) (layer "B.Cu") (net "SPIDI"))
 (segment (start 99.357693 75.235) (end 99.357693 74.6) (width 0.2) (layer "B.Cu") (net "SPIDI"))
 (segment (start 94.912693 73.33) (end 91.737693 76.505) (width 0.2) (layer "B.Cu") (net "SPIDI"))
 (segment (start 98.087693 73.33) (end 94.912693 73.33) (width 0.2) (layer "B.Cu") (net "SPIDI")))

